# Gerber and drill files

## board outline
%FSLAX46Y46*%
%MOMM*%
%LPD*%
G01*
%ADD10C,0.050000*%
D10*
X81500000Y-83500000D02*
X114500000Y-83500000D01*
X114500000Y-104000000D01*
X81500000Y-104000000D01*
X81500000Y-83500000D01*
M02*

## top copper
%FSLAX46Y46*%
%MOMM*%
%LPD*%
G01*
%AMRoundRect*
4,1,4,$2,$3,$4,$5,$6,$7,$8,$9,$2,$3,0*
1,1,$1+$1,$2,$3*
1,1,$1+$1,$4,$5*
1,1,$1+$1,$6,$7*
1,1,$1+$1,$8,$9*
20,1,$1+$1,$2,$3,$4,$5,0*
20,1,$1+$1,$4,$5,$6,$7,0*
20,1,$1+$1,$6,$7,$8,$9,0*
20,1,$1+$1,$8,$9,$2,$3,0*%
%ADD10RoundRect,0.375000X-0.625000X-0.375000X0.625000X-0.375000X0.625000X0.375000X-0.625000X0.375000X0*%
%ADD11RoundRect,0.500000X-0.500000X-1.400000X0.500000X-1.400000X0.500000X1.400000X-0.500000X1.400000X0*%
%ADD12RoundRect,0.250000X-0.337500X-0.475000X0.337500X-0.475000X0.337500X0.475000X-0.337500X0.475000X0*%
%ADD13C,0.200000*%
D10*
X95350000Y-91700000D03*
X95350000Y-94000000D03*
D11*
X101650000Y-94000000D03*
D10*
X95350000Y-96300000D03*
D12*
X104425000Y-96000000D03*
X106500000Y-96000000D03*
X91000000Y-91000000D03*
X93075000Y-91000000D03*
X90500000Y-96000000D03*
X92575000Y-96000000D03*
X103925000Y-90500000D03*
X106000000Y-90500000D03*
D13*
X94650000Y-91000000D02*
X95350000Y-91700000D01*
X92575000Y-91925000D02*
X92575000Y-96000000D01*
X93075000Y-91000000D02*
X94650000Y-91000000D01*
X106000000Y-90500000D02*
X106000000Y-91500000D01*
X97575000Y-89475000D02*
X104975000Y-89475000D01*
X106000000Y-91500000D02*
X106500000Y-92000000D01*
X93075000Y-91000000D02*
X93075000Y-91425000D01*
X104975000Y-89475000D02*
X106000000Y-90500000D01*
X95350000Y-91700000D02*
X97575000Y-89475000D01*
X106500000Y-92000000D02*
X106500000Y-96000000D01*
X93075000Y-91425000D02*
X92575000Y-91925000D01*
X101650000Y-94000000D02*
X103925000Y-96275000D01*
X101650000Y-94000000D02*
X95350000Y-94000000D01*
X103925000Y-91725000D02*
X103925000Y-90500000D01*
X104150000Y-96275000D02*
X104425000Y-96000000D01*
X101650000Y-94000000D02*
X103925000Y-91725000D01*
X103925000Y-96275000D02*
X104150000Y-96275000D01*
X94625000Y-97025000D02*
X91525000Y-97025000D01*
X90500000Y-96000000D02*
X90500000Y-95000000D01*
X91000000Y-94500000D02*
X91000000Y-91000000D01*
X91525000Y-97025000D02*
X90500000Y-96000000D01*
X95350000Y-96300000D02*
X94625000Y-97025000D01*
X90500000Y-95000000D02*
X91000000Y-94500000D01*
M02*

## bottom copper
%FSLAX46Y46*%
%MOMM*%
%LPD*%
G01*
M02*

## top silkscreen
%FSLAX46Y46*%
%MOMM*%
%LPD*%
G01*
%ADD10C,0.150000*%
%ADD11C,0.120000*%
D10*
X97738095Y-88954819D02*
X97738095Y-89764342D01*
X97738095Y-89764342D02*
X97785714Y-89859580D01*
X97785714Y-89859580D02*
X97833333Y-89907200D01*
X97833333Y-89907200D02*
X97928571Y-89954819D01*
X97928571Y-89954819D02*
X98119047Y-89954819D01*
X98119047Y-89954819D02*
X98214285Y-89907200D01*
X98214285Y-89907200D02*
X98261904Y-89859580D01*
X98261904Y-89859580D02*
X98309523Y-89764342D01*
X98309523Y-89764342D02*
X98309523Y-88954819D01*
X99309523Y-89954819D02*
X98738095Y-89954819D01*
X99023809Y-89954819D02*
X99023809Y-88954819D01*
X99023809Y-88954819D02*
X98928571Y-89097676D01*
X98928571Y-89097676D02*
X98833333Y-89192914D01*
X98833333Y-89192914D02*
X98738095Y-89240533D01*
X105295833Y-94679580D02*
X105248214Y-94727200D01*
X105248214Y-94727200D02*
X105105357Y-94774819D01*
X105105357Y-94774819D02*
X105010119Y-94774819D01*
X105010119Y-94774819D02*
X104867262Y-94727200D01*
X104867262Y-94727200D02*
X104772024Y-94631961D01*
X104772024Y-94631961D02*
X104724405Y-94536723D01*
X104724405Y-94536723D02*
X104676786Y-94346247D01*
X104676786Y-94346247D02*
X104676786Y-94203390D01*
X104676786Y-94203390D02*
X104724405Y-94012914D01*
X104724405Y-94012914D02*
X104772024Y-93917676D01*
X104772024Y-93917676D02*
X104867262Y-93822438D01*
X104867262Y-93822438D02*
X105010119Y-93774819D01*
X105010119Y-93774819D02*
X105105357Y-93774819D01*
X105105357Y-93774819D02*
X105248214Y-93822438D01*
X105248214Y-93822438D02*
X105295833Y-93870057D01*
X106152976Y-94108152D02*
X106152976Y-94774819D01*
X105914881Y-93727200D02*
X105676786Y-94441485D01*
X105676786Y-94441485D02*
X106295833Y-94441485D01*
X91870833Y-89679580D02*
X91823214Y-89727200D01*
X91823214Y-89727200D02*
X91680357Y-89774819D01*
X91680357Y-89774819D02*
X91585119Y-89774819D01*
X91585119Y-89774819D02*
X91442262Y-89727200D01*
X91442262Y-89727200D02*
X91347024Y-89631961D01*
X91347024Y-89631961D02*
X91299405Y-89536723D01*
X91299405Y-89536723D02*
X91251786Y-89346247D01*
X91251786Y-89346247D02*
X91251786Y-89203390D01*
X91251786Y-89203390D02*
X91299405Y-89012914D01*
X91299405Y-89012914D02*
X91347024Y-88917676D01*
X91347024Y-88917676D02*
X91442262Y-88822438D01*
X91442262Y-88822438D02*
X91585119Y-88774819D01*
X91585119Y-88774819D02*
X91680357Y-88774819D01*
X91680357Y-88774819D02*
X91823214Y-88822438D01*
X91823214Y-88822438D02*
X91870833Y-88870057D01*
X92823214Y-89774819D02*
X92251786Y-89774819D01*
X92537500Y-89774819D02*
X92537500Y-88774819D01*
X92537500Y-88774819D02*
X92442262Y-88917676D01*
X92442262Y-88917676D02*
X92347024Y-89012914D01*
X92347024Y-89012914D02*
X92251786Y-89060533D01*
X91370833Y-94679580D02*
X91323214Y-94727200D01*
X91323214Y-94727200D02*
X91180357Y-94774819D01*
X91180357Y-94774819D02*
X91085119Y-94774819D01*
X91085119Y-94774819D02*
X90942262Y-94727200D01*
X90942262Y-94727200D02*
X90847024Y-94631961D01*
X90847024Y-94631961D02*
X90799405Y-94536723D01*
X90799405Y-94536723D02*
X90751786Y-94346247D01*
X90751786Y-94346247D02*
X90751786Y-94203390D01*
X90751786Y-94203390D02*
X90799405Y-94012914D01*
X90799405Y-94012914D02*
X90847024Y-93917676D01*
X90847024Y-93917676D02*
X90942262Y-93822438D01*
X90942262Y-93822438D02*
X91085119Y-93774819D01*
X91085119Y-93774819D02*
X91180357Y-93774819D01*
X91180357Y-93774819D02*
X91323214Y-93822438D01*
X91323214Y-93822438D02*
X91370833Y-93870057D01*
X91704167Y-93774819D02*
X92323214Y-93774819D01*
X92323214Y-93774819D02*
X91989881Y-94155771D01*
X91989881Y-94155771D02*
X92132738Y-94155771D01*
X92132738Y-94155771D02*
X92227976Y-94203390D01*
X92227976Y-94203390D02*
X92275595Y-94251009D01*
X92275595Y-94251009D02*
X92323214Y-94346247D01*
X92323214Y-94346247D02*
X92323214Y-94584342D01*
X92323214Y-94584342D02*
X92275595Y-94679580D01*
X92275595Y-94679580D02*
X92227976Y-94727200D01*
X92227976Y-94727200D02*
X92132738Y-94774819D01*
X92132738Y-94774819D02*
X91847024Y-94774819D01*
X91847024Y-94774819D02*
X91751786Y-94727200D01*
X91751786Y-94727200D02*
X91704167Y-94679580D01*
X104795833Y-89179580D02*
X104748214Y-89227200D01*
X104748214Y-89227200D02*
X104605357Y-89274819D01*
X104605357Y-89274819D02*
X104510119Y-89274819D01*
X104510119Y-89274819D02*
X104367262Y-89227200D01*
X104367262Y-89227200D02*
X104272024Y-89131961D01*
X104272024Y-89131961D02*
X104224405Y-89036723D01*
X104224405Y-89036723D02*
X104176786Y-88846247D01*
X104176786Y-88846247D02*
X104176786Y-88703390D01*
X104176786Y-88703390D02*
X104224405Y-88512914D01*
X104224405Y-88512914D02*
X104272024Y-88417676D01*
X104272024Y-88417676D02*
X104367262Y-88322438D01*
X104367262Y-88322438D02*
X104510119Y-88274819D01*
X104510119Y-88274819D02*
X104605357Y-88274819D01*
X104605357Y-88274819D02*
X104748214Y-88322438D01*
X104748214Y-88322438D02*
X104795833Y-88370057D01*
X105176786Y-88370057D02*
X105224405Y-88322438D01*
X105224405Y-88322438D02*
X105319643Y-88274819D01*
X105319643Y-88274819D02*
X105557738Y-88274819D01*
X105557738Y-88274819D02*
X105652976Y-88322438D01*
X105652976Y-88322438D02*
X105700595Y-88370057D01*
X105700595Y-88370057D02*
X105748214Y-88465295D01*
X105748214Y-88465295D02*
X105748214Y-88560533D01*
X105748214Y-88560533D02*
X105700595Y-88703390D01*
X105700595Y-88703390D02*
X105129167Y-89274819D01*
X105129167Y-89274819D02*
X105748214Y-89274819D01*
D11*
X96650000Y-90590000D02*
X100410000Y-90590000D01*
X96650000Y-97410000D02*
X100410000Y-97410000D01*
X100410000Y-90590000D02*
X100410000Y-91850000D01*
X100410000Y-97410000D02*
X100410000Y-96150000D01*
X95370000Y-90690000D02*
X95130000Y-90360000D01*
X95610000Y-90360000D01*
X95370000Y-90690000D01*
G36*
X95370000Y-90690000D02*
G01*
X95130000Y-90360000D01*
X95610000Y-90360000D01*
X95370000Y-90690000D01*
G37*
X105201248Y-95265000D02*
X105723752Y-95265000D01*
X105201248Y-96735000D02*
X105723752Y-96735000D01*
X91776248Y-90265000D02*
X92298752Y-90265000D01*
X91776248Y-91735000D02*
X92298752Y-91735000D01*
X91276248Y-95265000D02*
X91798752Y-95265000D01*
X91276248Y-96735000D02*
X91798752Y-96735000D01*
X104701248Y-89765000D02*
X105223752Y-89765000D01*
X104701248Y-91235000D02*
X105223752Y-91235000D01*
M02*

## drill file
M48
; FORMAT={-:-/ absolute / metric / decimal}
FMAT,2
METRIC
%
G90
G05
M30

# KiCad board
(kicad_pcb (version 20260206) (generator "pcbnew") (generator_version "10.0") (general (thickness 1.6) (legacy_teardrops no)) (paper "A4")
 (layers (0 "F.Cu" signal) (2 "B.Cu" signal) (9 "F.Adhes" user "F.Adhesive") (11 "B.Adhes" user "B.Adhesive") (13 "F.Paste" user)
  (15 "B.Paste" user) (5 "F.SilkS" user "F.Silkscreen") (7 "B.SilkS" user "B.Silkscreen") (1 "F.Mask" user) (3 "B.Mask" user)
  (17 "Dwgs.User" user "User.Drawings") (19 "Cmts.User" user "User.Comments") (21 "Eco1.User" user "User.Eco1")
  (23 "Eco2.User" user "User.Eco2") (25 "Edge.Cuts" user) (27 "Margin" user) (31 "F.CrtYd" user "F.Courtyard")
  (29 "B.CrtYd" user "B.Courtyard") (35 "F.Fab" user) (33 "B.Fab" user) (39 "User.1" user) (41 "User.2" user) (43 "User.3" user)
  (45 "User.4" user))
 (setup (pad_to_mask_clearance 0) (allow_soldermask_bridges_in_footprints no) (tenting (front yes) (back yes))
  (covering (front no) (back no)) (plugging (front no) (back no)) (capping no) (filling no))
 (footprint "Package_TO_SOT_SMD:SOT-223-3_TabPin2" (layer "F.Cu") (at 98.5 94)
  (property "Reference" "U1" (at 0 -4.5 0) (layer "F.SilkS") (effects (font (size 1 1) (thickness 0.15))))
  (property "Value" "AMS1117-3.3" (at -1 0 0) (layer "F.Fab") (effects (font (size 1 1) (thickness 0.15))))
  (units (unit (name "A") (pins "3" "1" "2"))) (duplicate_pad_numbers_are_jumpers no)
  (fp_line (start -1.85 -3.41) (end 1.91 -3.41) (stroke (width 0.12) (type solid)) (layer "F.SilkS"))
  (fp_line (start -1.85 3.41) (end 1.91 3.41) (stroke (width 0.12) (type solid)) (layer "F.SilkS"))
  (fp_line (start 1.91 -3.41) (end 1.91 -2.15) (stroke (width 0.12) (type solid)) (layer "F.SilkS"))
  (fp_line (start 1.91 3.41) (end 1.91 2.15) (stroke (width 0.12) (type solid)) (layer "F.SilkS"))
  (fp_poly
   (pts (xy -3.13 -3.31) (xy -3.37 -3.64) (xy -2.89 -3.64) (xy -3.13 -3.31)) (stroke (width 0.12) (type solid)) (fill yes) (layer "F.SilkS"))
  (pad "1" smd roundrect (at -3.15 -2.3) (size 2 1.5) (layers "F.Cu" "F.Mask" "F.Paste") (roundrect_rratio 0.25) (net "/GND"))
  (pad "2" smd roundrect (at -3.15 0) (size 2 1.5) (layers "F.Cu" "F.Mask" "F.Paste") (roundrect_rratio 0.25) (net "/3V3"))
  (pad "2" smd roundrect (at 3.15 0) (size 2 3.8) (layers "F.Cu" "F.Mask" "F.Paste") (roundrect_rratio 0.25) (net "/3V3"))
  (pad "3" smd roundrect (at -3.15 2.3) (size 2 1.5) (layers "F.Cu" "F.Mask" "F.Paste") (roundrect_rratio 0.25) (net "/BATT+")))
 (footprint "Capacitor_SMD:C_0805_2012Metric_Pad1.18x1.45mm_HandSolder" (layer "F.Cu") (at 105.4625 96)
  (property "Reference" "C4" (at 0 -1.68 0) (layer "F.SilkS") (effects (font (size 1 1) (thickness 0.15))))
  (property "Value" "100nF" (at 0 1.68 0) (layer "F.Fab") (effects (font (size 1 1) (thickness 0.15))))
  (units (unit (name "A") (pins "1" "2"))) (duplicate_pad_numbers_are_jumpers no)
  (fp_line (start -0.261252 -0.735) (end 0.261252 -0.735) (stroke (width 0.12) (type solid)) (layer "F.SilkS"))
  (fp_line (start -0.261252 0.735) (end 0.261252 0.735) (stroke (width 0.12) (type solid)) (layer "F.SilkS"))
  (pad "1" smd roundrect (at -1.0375 0) (size 1.175 1.45) (layers "F.Cu" "F.Mask" "F.Paste") (roundrect_rratio 0.212766) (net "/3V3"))
  (pad "2" smd roundrect (at 1.0375 0) (size 1.175 1.45) (layers "F.Cu" "F.Mask" "F.Paste") (roundrect_rratio 0.212766) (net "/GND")))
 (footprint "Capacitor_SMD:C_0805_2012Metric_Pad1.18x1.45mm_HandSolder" (layer "F.Cu") (at 92.0375 91)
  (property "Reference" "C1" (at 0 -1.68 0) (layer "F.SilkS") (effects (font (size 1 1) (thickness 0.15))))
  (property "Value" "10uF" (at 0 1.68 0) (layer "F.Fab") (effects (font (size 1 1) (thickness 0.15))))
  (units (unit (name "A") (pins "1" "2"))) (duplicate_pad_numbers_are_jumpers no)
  (fp_line (start -0.261252 -0.735) (end 0.261252 -0.735) (stroke (width 0.12) (type solid)) (layer "F.SilkS"))
  (fp_line (start -0.261252 0.735) (end 0.261252 0.735) (stroke (width 0.12) (type solid)) (layer "F.SilkS"))
  (pad "1" smd roundrect (at -1.0375 0) (size 1.175 1.45) (layers "F.Cu" "F.Mask" "F.Paste") (roundrect_rratio 0.212766) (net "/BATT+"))
  (pad "2" smd roundrect (at 1.0375 0) (size 1.175 1.45) (layers "F.Cu" "F.Mask" "F.Paste") (roundrect_rratio 0.212766) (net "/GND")))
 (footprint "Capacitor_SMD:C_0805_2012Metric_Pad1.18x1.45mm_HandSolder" (layer "F.Cu") (at 91.5375 96)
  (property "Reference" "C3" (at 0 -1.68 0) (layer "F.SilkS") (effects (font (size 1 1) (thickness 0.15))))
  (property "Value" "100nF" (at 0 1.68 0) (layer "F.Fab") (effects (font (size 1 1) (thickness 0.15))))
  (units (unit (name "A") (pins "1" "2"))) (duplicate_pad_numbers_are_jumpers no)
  (fp_line (start -0.261252 -0.735) (end 0.261252 -0.735) (stroke (width 0.12) (type solid)) (layer "F.SilkS"))
  (fp_line (start -0.261252 0.735) (end 0.261252 0.735) (stroke (width 0.12) (type solid)) (layer "F.SilkS"))
  (pad "1" smd roundrect (at -1.0375 0) (size 1.175 1.45) (layers "F.Cu" "F.Mask" "F.Paste") (roundrect_rratio 0.212766) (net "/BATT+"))
  (pad "2" smd roundrect (at 1.0375 0) (size 1.175 1.45) (layers "F.Cu" "F.Mask" "F.Paste") (roundrect_rratio 0.212766) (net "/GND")))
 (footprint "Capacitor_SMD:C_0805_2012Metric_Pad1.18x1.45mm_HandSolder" (layer "F.Cu") (at 104.9625 90.5)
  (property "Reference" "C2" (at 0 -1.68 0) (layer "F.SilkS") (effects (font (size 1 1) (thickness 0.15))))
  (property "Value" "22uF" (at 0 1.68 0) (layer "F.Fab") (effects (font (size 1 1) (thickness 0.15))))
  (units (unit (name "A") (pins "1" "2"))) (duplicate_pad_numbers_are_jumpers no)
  (fp_line (start -0.261252 -0.735) (end 0.261252 -0.735) (stroke (width 0.12) (type solid)) (layer "F.SilkS"))
  (fp_line (start -0.261252 0.735) (end 0.261252 0.735) (stroke (width 0.12) (type solid)) (layer "F.SilkS"))
  (pad "1" smd roundrect (at -1.0375 0) (size 1.175 1.45) (layers "F.Cu" "F.Mask" "F.Paste") (roundrect_rratio 0.212766) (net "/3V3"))
  (pad "2" smd roundrect (at 1.0375 0) (size 1.175 1.45) (layers "F.Cu" "F.Mask" "F.Paste") (roundrect_rratio 0.212766) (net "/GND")))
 (gr_rect (start 81.5 83.5) (end 114.5 104) (stroke (width 0.05) (type default)) (fill no) (layer "Edge.Cuts"))
 (segment (start 94.65 91) (end 95.35 91.7) (width 0.2) (layer "F.Cu") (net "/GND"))
 (segment (start 92.575 91.925) (end 92.575 96) (width 0.2) (layer "F.Cu") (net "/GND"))
 (segment (start 93.075 91) (end 94.65 91) (width 0.2) (layer "F.Cu") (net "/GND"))
 (segment (start 106 90.5) (end 106 91.5) (width 0.2) (layer "F.Cu") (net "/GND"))
 (segment (start 97.575 89.475) (end 104.975 89.475) (width 0.2) (layer "F.Cu") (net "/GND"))
 (segment (start 106 91.5) (end 106.5 92) (width 0.2) (layer "F.Cu") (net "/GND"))
 (segment (start 93.075 91) (end 93.075 91.425) (width 0.2) (layer "F.Cu") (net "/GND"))
 (segment (start 104.975 89.475) (end 106 90.5) (width 0.2) (layer "F.Cu") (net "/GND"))
 (segment (start 95.35 91.7) (end 97.575 89.475) (width 0.2) (layer "F.Cu") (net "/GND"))
 (segment (start 106.5 92) (end 106.5 96) (width 0.2) (layer "F.Cu") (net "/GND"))
 (segment (start 93.075 91.425) (end 92.575 91.925) (width 0.2) (layer "F.Cu") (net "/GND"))
 (segment (start 101.65 94) (end 103.925 96.275) (width 0.2) (layer "F.Cu") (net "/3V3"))
 (segment (start 101.65 94) (end 95.35 94) (width 0.2) (layer "F.Cu") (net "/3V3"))
 (segment (start 103.925 91.725) (end 103.925 90.5) (width 0.2) (layer "F.Cu") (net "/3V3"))
 (segment (start 104.15 96.275) (end 104.425 96) (width 0.2) (layer "F.Cu") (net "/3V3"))
 (segment (start 101.65 94) (end 103.925 91.725) (width 0.2) (layer "F.Cu") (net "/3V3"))
 (segment (start 103.925 96.275) (end 104.15 96.275) (width 0.2) (layer "F.Cu") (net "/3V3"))
 (segment (start 94.625 97.025) (end 91.525 97.025) (width 0.2) (layer "F.Cu") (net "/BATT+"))
 (segment (start 90.5 96) (end 90.5 95) (width 0.2) (layer "F.Cu") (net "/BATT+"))
 (segment (start 91 94.5) (end 91 91) (width 0.2) (layer "F.Cu") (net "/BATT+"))
 (segment (start 91.525 97.025) (end 90.5 96) (width 0.2) (layer "F.Cu") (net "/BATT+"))
 (segment (start 95.35 96.3) (end 94.625 97.025) (width 0.2) (layer "F.Cu") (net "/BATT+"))
 (segment (start 90.5 95) (end 91 94.5) (width 0.2) (layer "F.Cu") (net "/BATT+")))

